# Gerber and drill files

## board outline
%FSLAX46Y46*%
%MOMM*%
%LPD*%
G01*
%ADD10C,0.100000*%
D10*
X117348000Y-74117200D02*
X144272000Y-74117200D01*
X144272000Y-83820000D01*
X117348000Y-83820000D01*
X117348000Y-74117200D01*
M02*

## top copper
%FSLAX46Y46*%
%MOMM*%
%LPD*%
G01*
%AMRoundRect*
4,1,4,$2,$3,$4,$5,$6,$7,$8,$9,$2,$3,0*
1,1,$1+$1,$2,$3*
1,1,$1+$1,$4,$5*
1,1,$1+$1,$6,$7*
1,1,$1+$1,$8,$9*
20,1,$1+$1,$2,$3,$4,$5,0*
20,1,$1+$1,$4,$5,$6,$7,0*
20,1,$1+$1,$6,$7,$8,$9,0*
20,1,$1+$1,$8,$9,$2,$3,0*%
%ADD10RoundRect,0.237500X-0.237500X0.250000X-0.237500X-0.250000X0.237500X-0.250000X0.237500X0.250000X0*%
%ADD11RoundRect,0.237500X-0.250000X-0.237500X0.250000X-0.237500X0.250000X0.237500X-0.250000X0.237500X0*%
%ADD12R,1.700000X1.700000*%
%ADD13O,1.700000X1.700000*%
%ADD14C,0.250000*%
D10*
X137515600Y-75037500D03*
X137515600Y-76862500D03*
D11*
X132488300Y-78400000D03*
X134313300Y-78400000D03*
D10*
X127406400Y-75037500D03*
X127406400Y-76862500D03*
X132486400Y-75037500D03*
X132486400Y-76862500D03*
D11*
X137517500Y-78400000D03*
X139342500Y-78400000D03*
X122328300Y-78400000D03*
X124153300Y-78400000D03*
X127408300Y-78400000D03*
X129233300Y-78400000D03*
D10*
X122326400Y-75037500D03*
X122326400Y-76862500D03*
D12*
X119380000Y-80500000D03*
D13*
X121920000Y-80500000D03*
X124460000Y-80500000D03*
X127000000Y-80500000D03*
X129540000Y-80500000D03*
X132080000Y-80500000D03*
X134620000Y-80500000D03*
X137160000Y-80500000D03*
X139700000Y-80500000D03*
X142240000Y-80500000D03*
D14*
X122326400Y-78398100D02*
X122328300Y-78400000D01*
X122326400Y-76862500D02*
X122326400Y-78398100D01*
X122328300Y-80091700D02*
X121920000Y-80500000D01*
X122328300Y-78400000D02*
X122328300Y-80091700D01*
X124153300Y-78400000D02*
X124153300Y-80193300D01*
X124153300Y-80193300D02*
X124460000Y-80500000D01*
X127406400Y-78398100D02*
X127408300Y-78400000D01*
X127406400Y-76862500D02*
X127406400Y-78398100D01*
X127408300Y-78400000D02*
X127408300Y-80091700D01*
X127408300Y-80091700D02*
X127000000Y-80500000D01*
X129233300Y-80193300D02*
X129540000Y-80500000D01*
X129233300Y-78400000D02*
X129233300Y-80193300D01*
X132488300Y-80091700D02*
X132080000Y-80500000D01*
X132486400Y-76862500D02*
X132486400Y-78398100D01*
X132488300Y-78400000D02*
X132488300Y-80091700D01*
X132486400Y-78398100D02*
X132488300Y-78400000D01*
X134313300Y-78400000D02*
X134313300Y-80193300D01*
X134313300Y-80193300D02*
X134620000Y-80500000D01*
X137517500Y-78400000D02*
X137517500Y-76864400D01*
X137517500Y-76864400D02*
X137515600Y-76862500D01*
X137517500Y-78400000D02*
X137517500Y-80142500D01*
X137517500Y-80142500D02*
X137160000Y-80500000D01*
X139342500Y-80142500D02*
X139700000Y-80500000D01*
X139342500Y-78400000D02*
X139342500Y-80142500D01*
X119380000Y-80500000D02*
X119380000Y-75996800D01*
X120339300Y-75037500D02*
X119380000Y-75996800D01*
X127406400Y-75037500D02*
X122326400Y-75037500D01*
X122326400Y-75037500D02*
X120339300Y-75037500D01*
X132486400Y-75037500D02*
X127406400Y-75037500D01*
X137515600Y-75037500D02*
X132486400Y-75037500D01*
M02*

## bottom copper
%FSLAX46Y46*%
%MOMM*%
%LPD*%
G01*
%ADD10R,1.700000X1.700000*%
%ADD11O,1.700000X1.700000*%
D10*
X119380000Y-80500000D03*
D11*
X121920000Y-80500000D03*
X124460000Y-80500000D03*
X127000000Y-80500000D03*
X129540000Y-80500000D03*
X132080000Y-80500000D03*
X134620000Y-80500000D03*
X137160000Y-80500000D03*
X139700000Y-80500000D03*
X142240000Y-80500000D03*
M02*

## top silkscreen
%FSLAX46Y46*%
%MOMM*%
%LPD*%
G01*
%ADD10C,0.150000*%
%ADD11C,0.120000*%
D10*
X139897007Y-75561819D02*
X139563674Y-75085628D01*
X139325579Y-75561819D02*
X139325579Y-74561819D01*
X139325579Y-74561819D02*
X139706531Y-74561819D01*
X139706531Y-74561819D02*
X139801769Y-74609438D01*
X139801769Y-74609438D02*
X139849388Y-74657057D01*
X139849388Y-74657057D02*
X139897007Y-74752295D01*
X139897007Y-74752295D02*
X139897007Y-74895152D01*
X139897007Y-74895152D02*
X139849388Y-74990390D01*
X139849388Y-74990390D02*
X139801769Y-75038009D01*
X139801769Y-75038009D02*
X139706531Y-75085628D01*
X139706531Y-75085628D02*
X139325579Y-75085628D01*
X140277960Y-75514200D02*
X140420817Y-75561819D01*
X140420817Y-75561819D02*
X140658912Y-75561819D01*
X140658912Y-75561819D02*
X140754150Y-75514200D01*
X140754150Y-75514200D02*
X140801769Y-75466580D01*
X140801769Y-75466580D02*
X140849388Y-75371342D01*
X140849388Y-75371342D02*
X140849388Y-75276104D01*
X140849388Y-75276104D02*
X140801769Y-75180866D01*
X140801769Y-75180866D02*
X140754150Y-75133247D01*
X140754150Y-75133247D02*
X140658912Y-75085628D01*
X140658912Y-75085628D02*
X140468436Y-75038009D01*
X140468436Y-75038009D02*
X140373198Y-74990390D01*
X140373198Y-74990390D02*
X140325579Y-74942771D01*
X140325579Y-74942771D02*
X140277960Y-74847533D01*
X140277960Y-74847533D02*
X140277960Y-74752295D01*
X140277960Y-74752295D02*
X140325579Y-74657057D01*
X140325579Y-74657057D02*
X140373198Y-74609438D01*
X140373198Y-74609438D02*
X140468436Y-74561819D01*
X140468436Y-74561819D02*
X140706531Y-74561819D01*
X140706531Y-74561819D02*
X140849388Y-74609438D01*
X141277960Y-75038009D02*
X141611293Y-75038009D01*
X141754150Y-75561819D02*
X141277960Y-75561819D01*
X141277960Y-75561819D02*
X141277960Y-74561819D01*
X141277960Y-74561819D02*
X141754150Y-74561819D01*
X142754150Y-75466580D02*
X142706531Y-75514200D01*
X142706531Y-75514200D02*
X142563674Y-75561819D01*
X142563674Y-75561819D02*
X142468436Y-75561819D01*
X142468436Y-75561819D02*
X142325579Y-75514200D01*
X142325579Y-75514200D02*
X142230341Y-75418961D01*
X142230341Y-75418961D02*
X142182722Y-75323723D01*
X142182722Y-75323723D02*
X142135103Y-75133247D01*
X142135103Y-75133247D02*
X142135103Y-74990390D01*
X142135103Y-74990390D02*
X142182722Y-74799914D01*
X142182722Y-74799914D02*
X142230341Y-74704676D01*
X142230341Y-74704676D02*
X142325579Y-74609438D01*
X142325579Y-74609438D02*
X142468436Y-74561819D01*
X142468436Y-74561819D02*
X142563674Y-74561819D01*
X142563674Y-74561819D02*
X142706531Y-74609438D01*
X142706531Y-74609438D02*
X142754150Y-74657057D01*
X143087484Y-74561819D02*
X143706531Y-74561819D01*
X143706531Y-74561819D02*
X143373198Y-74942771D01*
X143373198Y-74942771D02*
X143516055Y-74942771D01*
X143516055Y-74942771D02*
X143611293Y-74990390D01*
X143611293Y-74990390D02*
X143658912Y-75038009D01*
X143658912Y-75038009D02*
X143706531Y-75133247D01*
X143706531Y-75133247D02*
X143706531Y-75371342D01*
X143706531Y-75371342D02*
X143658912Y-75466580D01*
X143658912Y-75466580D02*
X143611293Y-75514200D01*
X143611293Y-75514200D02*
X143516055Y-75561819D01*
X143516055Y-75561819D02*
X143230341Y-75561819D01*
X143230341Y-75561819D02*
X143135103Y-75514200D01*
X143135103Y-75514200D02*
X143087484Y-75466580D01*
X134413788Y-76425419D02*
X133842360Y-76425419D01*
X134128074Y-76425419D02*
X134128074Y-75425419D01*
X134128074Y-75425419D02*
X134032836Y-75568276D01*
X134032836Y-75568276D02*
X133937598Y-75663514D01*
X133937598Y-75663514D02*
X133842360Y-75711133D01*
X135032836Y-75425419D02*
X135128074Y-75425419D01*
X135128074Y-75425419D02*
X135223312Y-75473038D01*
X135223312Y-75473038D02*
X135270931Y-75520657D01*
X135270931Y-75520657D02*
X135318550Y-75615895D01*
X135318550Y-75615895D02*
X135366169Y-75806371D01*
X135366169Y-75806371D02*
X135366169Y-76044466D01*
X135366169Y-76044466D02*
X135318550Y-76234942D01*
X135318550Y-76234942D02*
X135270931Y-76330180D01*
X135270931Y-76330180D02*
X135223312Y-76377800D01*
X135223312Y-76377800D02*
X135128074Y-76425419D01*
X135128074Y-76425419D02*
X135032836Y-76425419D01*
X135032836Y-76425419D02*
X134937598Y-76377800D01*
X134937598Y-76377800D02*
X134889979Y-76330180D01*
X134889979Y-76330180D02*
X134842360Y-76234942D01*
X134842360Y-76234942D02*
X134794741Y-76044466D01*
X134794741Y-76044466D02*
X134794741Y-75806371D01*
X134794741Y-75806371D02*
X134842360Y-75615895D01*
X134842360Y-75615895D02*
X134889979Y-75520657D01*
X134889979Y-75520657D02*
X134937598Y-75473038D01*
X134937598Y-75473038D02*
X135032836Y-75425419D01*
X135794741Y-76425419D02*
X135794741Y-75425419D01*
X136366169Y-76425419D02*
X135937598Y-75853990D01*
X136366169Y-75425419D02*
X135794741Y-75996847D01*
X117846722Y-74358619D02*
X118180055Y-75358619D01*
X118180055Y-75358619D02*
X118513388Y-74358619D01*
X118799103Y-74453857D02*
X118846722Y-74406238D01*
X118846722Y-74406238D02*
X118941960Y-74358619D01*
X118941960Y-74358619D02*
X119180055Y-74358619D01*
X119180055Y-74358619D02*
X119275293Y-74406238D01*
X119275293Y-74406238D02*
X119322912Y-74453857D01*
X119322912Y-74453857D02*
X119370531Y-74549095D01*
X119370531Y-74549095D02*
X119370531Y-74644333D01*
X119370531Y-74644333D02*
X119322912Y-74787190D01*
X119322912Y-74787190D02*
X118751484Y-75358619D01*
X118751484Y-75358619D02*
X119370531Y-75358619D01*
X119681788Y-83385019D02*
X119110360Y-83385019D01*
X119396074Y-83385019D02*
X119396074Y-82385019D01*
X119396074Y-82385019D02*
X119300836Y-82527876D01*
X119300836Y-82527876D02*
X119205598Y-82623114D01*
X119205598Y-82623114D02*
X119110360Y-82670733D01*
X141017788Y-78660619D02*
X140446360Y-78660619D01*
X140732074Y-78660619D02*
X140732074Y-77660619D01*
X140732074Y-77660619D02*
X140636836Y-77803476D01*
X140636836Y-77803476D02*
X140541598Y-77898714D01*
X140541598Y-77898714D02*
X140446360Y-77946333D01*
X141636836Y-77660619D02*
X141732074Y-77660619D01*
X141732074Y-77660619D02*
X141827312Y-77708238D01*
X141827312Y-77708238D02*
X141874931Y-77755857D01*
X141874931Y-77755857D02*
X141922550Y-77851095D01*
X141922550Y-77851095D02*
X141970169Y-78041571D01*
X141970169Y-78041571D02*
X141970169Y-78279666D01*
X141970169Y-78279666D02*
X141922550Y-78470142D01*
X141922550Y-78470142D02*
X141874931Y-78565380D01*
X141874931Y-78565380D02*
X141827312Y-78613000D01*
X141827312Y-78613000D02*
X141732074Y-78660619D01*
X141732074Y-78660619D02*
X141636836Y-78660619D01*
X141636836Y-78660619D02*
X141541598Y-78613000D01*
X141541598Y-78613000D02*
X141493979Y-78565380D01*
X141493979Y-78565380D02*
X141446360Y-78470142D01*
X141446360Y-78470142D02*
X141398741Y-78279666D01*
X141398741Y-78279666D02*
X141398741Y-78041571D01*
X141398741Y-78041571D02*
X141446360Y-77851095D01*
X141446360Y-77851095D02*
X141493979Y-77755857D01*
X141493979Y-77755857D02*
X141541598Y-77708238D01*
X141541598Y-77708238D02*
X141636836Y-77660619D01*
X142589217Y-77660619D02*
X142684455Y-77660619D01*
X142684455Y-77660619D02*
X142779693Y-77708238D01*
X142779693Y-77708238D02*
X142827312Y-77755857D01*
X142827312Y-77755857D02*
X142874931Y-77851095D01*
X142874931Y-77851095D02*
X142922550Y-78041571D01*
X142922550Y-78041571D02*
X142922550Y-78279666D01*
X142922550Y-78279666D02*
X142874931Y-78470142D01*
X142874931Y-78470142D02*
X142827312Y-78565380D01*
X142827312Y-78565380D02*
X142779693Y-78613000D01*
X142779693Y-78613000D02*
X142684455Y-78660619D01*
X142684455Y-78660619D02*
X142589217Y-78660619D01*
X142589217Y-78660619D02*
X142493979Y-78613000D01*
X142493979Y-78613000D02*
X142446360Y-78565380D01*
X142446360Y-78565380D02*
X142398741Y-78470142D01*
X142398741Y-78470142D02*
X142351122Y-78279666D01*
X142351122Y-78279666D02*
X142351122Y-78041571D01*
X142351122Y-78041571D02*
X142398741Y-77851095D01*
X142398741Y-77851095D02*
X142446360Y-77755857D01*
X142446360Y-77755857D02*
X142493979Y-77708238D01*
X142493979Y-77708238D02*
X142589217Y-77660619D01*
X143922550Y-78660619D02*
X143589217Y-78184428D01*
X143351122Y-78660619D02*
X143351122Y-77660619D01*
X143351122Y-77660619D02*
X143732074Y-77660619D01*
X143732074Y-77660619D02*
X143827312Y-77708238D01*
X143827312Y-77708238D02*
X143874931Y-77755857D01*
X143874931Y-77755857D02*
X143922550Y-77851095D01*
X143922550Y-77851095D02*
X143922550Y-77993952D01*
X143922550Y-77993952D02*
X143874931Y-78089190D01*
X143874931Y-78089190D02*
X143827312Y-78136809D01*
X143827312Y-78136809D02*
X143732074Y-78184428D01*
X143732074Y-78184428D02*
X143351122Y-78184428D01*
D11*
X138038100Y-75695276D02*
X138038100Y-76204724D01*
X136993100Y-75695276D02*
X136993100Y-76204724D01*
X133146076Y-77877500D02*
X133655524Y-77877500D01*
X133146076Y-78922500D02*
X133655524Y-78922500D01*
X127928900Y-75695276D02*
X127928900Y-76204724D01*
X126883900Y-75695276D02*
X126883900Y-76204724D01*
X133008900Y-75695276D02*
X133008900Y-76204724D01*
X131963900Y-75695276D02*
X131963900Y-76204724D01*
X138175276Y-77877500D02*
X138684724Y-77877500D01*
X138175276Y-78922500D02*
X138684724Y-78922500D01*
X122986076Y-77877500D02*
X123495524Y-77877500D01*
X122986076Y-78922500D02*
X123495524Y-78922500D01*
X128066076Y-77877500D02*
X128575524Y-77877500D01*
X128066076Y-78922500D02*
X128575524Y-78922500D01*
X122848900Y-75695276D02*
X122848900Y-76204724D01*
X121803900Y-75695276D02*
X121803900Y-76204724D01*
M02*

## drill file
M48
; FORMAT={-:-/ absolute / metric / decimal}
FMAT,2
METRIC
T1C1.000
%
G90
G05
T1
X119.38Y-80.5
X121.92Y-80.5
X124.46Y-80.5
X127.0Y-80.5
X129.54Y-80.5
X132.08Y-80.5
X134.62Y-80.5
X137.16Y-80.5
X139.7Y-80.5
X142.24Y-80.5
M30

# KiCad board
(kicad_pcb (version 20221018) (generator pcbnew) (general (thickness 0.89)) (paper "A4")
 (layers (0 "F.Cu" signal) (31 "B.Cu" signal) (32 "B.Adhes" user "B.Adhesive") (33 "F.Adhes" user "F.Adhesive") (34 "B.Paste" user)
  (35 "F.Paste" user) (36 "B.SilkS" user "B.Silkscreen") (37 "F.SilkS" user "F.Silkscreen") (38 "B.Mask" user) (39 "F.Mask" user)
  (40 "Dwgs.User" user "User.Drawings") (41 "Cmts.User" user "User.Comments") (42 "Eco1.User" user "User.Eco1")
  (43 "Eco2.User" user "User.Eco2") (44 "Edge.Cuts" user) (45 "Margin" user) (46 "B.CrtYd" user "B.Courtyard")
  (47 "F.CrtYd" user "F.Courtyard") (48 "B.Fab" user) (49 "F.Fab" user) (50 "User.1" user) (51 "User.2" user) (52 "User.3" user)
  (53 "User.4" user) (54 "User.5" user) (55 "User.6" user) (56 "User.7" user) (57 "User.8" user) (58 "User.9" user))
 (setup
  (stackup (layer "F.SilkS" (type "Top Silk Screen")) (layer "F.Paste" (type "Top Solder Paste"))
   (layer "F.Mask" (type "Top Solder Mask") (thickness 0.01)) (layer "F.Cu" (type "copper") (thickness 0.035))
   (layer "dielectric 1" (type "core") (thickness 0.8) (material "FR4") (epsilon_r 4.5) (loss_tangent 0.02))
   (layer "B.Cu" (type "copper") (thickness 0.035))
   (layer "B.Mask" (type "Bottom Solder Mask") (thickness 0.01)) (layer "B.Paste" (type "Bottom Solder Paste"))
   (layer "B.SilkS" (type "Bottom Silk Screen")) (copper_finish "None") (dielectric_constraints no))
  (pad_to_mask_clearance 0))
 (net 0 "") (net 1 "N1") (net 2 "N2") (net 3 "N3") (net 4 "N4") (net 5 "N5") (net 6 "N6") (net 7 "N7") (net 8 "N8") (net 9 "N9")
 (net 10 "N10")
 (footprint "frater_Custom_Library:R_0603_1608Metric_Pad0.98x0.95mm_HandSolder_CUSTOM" (layer "F.Cu") (at 137.5156 75.95 -90)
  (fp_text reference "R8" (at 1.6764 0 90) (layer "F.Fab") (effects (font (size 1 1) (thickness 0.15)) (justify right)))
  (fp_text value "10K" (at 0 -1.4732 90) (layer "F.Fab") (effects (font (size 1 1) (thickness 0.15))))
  (fp_line (start -0.254724 -0.5225) (end 0.254724 -0.5225) (stroke (width 0.12) (type solid)) (layer "F.SilkS"))
  (fp_line (start -0.254724 0.5225) (end 0.254724 0.5225) (stroke (width 0.12) (type solid)) (layer "F.SilkS"))
  (pad "1" smd roundrect (at -0.9125 0 270) (size 0.975 0.95) (layers "F.Cu" "F.Paste" "F.Mask") (roundrect_rratio 0.25) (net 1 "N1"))
  (pad "2" smd roundrect (at 0.9125 0 270) (size 0.975 0.95) (layers "F.Cu" "F.Paste" "F.Mask") (roundrect_rratio 0.25) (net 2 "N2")))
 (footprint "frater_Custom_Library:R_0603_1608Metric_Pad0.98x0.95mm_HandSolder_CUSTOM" (layer "F.Cu") (at 133.4008 78.4)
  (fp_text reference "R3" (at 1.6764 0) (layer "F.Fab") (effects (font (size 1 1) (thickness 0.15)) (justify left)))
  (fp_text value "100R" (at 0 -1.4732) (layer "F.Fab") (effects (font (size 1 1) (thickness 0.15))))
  (fp_line (start -0.254724 -0.5225) (end 0.254724 -0.5225) (stroke (width 0.12) (type solid)) (layer "F.SilkS"))
  (fp_line (start -0.254724 0.5225) (end 0.254724 0.5225) (stroke (width 0.12) (type solid)) (layer "F.SilkS"))
  (pad "1" smd roundrect (at -0.9125 0) (size 0.975 0.95) (layers "F.Cu" "F.Paste" "F.Mask") (roundrect_rratio 0.25) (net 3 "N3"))
  (pad "2" smd roundrect (at 0.9125 0) (size 0.975 0.95) (layers "F.Cu" "F.Paste" "F.Mask") (roundrect_rratio 0.25) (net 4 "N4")))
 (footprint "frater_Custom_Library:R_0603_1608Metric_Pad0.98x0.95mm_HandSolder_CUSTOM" (layer "F.Cu") (at 127.4064 75.95 -90)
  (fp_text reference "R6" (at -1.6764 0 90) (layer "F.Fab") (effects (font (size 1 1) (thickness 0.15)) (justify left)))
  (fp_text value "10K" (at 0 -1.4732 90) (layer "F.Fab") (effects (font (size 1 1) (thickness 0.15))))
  (fp_line (start -0.254724 -0.5225) (end 0.254724 -0.5225) (stroke (width 0.12) (type solid)) (layer "F.SilkS"))
  (fp_line (start -0.254724 0.5225) (end 0.254724 0.5225) (stroke (width 0.12) (type solid)) (layer "F.SilkS"))
  (pad "1" smd roundrect (at -0.9125 0 270) (size 0.975 0.95) (layers "F.Cu" "F.Paste" "F.Mask") (roundrect_rratio 0.25) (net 1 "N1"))
  (pad "2" smd roundrect (at 0.9125 0 270) (size 0.975 0.95) (layers "F.Cu" "F.Paste" "F.Mask") (roundrect_rratio 0.25) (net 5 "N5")))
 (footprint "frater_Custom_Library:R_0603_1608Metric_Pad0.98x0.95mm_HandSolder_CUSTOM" (layer "F.Cu") (at 132.4864 75.95 -90)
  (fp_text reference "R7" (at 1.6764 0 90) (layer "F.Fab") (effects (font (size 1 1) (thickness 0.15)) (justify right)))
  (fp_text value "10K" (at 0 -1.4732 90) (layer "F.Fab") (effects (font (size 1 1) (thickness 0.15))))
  (fp_line (start -0.254724 -0.5225) (end 0.254724 -0.5225) (stroke (width 0.12) (type solid)) (layer "F.SilkS"))
  (fp_line (start -0.254724 0.5225) (end 0.254724 0.5225) (stroke (width 0.12) (type solid)) (layer "F.SilkS"))
  (pad "1" smd roundrect (at -0.9125 0 270) (size 0.975 0.95) (layers "F.Cu" "F.Paste" "F.Mask") (roundrect_rratio 0.25) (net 1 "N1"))
  (pad "2" smd roundrect (at 0.9125 0 270) (size 0.975 0.95) (layers "F.Cu" "F.Paste" "F.Mask") (roundrect_rratio 0.25) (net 3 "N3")))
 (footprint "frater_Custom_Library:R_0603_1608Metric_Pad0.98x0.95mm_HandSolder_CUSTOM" (layer "F.Cu") (at 138.43 78.4)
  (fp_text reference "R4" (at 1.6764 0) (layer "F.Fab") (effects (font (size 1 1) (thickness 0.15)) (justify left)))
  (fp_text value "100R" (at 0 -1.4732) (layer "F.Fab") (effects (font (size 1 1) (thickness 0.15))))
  (fp_line (start -0.254724 -0.5225) (end 0.254724 -0.5225) (stroke (width 0.12) (type solid)) (layer "F.SilkS"))
  (fp_line (start -0.254724 0.5225) (end 0.254724 0.5225) (stroke (width 0.12) (type solid)) (layer "F.SilkS"))
  (pad "1" smd roundrect (at -0.9125 0) (size 0.975 0.95) (layers "F.Cu" "F.Paste" "F.Mask") (roundrect_rratio 0.25) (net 2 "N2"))
  (pad "2" smd roundrect (at 0.9125 0) (size 0.975 0.95) (layers "F.Cu" "F.Paste" "F.Mask") (roundrect_rratio 0.25) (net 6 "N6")))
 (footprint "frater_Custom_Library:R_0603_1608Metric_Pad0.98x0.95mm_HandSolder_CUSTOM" (layer "F.Cu") (at 123.2408 78.4)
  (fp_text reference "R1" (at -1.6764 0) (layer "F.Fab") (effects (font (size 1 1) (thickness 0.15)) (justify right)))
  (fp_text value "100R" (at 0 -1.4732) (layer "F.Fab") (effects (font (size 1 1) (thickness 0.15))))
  (fp_line (start -0.254724 -0.5225) (end 0.254724 -0.5225) (stroke (width 0.12) (type solid)) (layer "F.SilkS"))
  (fp_line (start -0.254724 0.5225) (end 0.254724 0.5225) (stroke (width 0.12) (type solid)) (layer "F.SilkS"))
  (pad "1" smd roundrect (at -0.9125 0) (size 0.975 0.95) (layers "F.Cu" "F.Paste" "F.Mask") (roundrect_rratio 0.25) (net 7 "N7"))
  (pad "2" smd roundrect (at 0.9125 0) (size 0.975 0.95) (layers "F.Cu" "F.Paste" "F.Mask") (roundrect_rratio 0.25) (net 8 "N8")))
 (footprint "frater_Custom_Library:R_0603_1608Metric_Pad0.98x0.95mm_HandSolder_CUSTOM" (layer "F.Cu") (at 128.3208 78.4)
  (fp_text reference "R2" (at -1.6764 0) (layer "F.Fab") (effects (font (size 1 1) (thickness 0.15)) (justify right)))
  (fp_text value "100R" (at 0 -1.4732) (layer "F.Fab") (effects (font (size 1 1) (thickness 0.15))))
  (fp_line (start -0.254724 -0.5225) (end 0.254724 -0.5225) (stroke (width 0.12) (type solid)) (layer "F.SilkS"))
  (fp_line (start -0.254724 0.5225) (end 0.254724 0.5225) (stroke (width 0.12) (type solid)) (layer "F.SilkS"))
  (pad "1" smd roundrect (at -0.9125 0) (size 0.975 0.95) (layers "F.Cu" "F.Paste" "F.Mask") (roundrect_rratio 0.25) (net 5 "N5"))
  (pad "2" smd roundrect (at 0.9125 0) (size 0.975 0.95) (layers "F.Cu" "F.Paste" "F.Mask") (roundrect_rratio 0.25) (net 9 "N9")))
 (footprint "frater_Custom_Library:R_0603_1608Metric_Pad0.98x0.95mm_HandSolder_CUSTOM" (layer "F.Cu") (at 122.3264 75.95 -90)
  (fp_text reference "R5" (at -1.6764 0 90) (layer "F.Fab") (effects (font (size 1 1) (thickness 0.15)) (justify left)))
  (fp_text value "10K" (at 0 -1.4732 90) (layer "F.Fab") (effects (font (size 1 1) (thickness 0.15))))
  (fp_line (start -0.254724 -0.5225) (end 0.254724 -0.5225) (stroke (width 0.12) (type solid)) (layer "F.SilkS"))
  (fp_line (start -0.254724 0.5225) (end 0.254724 0.5225) (stroke (width 0.12) (type solid)) (layer "F.SilkS"))
  (pad "1" smd roundrect (at -0.9125 0 270) (size 0.975 0.95) (layers "F.Cu" "F.Paste" "F.Mask") (roundrect_rratio 0.25) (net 1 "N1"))
  (pad "2" smd roundrect (at 0.9125 0 270) (size 0.975 0.95) (layers "F.Cu" "F.Paste" "F.Mask") (roundrect_rratio 0.25) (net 7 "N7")))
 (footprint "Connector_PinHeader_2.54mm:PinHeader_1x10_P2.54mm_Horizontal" (layer "B.Cu") (at 119.38 80.5 -90)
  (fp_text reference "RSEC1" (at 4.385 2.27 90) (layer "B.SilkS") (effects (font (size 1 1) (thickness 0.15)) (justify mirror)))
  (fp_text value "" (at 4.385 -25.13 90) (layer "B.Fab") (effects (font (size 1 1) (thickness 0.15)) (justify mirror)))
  (pad "1" thru_hole rect (at 0 0 270) (size 1.7 1.7) (drill 1) (layers "*.Cu" "*.Mask") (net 1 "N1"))
  (pad "2" thru_hole oval (at 0 -2.54 270) (size 1.7 1.7) (drill 1) (layers "*.Cu" "*.Mask") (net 7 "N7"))
  (pad "3" thru_hole oval (at 0 -5.08 270) (size 1.7 1.7) (drill 1) (layers "*.Cu" "*.Mask") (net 8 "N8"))
  (pad "4" thru_hole oval (at 0 -7.62 270) (size 1.7 1.7) (drill 1) (layers "*.Cu" "*.Mask") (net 5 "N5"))
  (pad "5" thru_hole oval (at 0 -10.16 270) (size 1.7 1.7) (drill 1) (layers "*.Cu" "*.Mask") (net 9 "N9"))
  (pad "6" thru_hole oval (at 0 -12.7 270) (size 1.7 1.7) (drill 1) (layers "*.Cu" "*.Mask") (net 3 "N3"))
  (pad "7" thru_hole oval (at 0 -15.24 270) (size 1.7 1.7) (drill 1) (layers "*.Cu" "*.Mask") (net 4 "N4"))
  (pad "8" thru_hole oval (at 0 -17.78 270) (size 1.7 1.7) (drill 1) (layers "*.Cu" "*.Mask") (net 2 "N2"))
  (pad "9" thru_hole oval (at 0 -20.32 270) (size 1.7 1.7) (drill 1) (layers "*.Cu" "*.Mask") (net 6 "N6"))
  (pad "10" thru_hole oval (at 0 -22.86 270) (size 1.7 1.7) (drill 1) (layers "*.Cu" "*.Mask") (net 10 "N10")))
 (gr_rect (start 117.348 74.1172) (end 144.272 83.82) (stroke (width 0.1) (type default)) (fill none) (layer "Edge.Cuts"))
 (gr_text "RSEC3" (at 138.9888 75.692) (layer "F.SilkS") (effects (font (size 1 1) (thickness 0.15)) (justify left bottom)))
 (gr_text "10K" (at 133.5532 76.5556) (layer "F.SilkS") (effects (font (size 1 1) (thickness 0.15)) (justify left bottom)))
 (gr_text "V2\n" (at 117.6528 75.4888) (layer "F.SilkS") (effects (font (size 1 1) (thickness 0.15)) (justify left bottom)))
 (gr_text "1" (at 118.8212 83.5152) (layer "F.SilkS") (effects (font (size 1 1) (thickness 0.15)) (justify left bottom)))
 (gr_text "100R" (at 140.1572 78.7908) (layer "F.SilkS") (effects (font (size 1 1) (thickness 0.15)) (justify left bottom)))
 (segment (start 122.3264 78.3981) (end 122.3283 78.4) (width 0.25) (layer "F.Cu") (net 7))
 (segment (start 122.3264 76.8625) (end 122.3264 78.3981) (width 0.25) (layer "F.Cu") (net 7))
 (segment (start 122.3283 80.0917) (end 121.92 80.5) (width 0.25) (layer "F.Cu") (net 7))
 (segment (start 122.3283 78.4) (end 122.3283 80.0917) (width 0.25) (layer "F.Cu") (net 7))
 (segment (start 124.1533 78.4) (end 124.1533 80.1933) (width 0.25) (layer "F.Cu") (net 8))
 (segment (start 124.1533 80.1933) (end 124.46 80.5) (width 0.25) (layer "F.Cu") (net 8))
 (segment (start 127.4064 78.3981) (end 127.4083 78.4) (width 0.25) (layer "F.Cu") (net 5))
 (segment (start 127.4064 76.8625) (end 127.4064 78.3981) (width 0.25) (layer "F.Cu") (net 5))
 (segment (start 127.4083 78.4) (end 127.4083 80.0917) (width 0.25) (layer "F.Cu") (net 5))
 (segment (start 127.4083 80.0917) (end 127 80.5) (width 0.25) (layer "F.Cu") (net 5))
 (segment (start 129.2333 80.1933) (end 129.54 80.5) (width 0.25) (layer "F.Cu") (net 9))
 (segment (start 129.2333 78.4) (end 129.2333 80.1933) (width 0.25) (layer "F.Cu") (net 9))
 (segment (start 132.4883 80.0917) (end 132.08 80.5) (width 0.25) (layer "F.Cu") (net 3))
 (segment (start 132.4864 76.8625) (end 132.4864 78.3981) (width 0.25) (layer "F.Cu") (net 3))
 (segment (start 132.4883 78.4) (end 132.4883 80.0917) (width 0.25) (layer "F.Cu") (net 3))
 (segment (start 132.4864 78.3981) (end 132.4883 78.4) (width 0.25) (layer "F.Cu") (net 3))
 (segment (start 134.3133 78.4) (end 134.3133 80.1933) (width 0.25) (layer "F.Cu") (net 4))
 (segment (start 134.3133 80.1933) (end 134.62 80.5) (width 0.25) (layer "F.Cu") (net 4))
 (segment (start 137.5175 78.4) (end 137.5175 76.8644) (width 0.25) (layer "F.Cu") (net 2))
 (segment (start 137.5175 76.8644) (end 137.5156 76.8625) (width 0.25) (layer "F.Cu") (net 2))
 (segment (start 137.5175 78.4) (end 137.5175 80.1425) (width 0.25) (layer "F.Cu") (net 2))
 (segment (start 137.5175 80.1425) (end 137.16 80.5) (width 0.25) (layer "F.Cu") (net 2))
 (segment (start 139.3425 80.1425) (end 139.7 80.5) (width 0.25) (layer "F.Cu") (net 6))
 (segment (start 139.3425 78.4) (end 139.3425 80.1425) (width 0.25) (layer "F.Cu") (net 6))
 (segment (start 119.38 80.5) (end 119.38 75.9968) (width 0.25) (layer "F.Cu") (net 1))
 (segment (start 120.3393 75.0375) (end 119.38 75.9968) (width 0.25) (layer "F.Cu") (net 1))
 (segment (start 127.4064 75.0375) (end 122.3264 75.0375) (width 0.25) (layer "F.Cu") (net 1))
 (segment (start 122.3264 75.0375) (end 120.3393 75.0375) (width 0.25) (layer "F.Cu") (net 1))
 (segment (start 132.4864 75.0375) (end 127.4064 75.0375) (width 0.25) (layer "F.Cu") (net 1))
 (segment (start 137.5156 75.0375) (end 132.4864 75.0375) (width 0.25) (layer "F.Cu") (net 1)))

